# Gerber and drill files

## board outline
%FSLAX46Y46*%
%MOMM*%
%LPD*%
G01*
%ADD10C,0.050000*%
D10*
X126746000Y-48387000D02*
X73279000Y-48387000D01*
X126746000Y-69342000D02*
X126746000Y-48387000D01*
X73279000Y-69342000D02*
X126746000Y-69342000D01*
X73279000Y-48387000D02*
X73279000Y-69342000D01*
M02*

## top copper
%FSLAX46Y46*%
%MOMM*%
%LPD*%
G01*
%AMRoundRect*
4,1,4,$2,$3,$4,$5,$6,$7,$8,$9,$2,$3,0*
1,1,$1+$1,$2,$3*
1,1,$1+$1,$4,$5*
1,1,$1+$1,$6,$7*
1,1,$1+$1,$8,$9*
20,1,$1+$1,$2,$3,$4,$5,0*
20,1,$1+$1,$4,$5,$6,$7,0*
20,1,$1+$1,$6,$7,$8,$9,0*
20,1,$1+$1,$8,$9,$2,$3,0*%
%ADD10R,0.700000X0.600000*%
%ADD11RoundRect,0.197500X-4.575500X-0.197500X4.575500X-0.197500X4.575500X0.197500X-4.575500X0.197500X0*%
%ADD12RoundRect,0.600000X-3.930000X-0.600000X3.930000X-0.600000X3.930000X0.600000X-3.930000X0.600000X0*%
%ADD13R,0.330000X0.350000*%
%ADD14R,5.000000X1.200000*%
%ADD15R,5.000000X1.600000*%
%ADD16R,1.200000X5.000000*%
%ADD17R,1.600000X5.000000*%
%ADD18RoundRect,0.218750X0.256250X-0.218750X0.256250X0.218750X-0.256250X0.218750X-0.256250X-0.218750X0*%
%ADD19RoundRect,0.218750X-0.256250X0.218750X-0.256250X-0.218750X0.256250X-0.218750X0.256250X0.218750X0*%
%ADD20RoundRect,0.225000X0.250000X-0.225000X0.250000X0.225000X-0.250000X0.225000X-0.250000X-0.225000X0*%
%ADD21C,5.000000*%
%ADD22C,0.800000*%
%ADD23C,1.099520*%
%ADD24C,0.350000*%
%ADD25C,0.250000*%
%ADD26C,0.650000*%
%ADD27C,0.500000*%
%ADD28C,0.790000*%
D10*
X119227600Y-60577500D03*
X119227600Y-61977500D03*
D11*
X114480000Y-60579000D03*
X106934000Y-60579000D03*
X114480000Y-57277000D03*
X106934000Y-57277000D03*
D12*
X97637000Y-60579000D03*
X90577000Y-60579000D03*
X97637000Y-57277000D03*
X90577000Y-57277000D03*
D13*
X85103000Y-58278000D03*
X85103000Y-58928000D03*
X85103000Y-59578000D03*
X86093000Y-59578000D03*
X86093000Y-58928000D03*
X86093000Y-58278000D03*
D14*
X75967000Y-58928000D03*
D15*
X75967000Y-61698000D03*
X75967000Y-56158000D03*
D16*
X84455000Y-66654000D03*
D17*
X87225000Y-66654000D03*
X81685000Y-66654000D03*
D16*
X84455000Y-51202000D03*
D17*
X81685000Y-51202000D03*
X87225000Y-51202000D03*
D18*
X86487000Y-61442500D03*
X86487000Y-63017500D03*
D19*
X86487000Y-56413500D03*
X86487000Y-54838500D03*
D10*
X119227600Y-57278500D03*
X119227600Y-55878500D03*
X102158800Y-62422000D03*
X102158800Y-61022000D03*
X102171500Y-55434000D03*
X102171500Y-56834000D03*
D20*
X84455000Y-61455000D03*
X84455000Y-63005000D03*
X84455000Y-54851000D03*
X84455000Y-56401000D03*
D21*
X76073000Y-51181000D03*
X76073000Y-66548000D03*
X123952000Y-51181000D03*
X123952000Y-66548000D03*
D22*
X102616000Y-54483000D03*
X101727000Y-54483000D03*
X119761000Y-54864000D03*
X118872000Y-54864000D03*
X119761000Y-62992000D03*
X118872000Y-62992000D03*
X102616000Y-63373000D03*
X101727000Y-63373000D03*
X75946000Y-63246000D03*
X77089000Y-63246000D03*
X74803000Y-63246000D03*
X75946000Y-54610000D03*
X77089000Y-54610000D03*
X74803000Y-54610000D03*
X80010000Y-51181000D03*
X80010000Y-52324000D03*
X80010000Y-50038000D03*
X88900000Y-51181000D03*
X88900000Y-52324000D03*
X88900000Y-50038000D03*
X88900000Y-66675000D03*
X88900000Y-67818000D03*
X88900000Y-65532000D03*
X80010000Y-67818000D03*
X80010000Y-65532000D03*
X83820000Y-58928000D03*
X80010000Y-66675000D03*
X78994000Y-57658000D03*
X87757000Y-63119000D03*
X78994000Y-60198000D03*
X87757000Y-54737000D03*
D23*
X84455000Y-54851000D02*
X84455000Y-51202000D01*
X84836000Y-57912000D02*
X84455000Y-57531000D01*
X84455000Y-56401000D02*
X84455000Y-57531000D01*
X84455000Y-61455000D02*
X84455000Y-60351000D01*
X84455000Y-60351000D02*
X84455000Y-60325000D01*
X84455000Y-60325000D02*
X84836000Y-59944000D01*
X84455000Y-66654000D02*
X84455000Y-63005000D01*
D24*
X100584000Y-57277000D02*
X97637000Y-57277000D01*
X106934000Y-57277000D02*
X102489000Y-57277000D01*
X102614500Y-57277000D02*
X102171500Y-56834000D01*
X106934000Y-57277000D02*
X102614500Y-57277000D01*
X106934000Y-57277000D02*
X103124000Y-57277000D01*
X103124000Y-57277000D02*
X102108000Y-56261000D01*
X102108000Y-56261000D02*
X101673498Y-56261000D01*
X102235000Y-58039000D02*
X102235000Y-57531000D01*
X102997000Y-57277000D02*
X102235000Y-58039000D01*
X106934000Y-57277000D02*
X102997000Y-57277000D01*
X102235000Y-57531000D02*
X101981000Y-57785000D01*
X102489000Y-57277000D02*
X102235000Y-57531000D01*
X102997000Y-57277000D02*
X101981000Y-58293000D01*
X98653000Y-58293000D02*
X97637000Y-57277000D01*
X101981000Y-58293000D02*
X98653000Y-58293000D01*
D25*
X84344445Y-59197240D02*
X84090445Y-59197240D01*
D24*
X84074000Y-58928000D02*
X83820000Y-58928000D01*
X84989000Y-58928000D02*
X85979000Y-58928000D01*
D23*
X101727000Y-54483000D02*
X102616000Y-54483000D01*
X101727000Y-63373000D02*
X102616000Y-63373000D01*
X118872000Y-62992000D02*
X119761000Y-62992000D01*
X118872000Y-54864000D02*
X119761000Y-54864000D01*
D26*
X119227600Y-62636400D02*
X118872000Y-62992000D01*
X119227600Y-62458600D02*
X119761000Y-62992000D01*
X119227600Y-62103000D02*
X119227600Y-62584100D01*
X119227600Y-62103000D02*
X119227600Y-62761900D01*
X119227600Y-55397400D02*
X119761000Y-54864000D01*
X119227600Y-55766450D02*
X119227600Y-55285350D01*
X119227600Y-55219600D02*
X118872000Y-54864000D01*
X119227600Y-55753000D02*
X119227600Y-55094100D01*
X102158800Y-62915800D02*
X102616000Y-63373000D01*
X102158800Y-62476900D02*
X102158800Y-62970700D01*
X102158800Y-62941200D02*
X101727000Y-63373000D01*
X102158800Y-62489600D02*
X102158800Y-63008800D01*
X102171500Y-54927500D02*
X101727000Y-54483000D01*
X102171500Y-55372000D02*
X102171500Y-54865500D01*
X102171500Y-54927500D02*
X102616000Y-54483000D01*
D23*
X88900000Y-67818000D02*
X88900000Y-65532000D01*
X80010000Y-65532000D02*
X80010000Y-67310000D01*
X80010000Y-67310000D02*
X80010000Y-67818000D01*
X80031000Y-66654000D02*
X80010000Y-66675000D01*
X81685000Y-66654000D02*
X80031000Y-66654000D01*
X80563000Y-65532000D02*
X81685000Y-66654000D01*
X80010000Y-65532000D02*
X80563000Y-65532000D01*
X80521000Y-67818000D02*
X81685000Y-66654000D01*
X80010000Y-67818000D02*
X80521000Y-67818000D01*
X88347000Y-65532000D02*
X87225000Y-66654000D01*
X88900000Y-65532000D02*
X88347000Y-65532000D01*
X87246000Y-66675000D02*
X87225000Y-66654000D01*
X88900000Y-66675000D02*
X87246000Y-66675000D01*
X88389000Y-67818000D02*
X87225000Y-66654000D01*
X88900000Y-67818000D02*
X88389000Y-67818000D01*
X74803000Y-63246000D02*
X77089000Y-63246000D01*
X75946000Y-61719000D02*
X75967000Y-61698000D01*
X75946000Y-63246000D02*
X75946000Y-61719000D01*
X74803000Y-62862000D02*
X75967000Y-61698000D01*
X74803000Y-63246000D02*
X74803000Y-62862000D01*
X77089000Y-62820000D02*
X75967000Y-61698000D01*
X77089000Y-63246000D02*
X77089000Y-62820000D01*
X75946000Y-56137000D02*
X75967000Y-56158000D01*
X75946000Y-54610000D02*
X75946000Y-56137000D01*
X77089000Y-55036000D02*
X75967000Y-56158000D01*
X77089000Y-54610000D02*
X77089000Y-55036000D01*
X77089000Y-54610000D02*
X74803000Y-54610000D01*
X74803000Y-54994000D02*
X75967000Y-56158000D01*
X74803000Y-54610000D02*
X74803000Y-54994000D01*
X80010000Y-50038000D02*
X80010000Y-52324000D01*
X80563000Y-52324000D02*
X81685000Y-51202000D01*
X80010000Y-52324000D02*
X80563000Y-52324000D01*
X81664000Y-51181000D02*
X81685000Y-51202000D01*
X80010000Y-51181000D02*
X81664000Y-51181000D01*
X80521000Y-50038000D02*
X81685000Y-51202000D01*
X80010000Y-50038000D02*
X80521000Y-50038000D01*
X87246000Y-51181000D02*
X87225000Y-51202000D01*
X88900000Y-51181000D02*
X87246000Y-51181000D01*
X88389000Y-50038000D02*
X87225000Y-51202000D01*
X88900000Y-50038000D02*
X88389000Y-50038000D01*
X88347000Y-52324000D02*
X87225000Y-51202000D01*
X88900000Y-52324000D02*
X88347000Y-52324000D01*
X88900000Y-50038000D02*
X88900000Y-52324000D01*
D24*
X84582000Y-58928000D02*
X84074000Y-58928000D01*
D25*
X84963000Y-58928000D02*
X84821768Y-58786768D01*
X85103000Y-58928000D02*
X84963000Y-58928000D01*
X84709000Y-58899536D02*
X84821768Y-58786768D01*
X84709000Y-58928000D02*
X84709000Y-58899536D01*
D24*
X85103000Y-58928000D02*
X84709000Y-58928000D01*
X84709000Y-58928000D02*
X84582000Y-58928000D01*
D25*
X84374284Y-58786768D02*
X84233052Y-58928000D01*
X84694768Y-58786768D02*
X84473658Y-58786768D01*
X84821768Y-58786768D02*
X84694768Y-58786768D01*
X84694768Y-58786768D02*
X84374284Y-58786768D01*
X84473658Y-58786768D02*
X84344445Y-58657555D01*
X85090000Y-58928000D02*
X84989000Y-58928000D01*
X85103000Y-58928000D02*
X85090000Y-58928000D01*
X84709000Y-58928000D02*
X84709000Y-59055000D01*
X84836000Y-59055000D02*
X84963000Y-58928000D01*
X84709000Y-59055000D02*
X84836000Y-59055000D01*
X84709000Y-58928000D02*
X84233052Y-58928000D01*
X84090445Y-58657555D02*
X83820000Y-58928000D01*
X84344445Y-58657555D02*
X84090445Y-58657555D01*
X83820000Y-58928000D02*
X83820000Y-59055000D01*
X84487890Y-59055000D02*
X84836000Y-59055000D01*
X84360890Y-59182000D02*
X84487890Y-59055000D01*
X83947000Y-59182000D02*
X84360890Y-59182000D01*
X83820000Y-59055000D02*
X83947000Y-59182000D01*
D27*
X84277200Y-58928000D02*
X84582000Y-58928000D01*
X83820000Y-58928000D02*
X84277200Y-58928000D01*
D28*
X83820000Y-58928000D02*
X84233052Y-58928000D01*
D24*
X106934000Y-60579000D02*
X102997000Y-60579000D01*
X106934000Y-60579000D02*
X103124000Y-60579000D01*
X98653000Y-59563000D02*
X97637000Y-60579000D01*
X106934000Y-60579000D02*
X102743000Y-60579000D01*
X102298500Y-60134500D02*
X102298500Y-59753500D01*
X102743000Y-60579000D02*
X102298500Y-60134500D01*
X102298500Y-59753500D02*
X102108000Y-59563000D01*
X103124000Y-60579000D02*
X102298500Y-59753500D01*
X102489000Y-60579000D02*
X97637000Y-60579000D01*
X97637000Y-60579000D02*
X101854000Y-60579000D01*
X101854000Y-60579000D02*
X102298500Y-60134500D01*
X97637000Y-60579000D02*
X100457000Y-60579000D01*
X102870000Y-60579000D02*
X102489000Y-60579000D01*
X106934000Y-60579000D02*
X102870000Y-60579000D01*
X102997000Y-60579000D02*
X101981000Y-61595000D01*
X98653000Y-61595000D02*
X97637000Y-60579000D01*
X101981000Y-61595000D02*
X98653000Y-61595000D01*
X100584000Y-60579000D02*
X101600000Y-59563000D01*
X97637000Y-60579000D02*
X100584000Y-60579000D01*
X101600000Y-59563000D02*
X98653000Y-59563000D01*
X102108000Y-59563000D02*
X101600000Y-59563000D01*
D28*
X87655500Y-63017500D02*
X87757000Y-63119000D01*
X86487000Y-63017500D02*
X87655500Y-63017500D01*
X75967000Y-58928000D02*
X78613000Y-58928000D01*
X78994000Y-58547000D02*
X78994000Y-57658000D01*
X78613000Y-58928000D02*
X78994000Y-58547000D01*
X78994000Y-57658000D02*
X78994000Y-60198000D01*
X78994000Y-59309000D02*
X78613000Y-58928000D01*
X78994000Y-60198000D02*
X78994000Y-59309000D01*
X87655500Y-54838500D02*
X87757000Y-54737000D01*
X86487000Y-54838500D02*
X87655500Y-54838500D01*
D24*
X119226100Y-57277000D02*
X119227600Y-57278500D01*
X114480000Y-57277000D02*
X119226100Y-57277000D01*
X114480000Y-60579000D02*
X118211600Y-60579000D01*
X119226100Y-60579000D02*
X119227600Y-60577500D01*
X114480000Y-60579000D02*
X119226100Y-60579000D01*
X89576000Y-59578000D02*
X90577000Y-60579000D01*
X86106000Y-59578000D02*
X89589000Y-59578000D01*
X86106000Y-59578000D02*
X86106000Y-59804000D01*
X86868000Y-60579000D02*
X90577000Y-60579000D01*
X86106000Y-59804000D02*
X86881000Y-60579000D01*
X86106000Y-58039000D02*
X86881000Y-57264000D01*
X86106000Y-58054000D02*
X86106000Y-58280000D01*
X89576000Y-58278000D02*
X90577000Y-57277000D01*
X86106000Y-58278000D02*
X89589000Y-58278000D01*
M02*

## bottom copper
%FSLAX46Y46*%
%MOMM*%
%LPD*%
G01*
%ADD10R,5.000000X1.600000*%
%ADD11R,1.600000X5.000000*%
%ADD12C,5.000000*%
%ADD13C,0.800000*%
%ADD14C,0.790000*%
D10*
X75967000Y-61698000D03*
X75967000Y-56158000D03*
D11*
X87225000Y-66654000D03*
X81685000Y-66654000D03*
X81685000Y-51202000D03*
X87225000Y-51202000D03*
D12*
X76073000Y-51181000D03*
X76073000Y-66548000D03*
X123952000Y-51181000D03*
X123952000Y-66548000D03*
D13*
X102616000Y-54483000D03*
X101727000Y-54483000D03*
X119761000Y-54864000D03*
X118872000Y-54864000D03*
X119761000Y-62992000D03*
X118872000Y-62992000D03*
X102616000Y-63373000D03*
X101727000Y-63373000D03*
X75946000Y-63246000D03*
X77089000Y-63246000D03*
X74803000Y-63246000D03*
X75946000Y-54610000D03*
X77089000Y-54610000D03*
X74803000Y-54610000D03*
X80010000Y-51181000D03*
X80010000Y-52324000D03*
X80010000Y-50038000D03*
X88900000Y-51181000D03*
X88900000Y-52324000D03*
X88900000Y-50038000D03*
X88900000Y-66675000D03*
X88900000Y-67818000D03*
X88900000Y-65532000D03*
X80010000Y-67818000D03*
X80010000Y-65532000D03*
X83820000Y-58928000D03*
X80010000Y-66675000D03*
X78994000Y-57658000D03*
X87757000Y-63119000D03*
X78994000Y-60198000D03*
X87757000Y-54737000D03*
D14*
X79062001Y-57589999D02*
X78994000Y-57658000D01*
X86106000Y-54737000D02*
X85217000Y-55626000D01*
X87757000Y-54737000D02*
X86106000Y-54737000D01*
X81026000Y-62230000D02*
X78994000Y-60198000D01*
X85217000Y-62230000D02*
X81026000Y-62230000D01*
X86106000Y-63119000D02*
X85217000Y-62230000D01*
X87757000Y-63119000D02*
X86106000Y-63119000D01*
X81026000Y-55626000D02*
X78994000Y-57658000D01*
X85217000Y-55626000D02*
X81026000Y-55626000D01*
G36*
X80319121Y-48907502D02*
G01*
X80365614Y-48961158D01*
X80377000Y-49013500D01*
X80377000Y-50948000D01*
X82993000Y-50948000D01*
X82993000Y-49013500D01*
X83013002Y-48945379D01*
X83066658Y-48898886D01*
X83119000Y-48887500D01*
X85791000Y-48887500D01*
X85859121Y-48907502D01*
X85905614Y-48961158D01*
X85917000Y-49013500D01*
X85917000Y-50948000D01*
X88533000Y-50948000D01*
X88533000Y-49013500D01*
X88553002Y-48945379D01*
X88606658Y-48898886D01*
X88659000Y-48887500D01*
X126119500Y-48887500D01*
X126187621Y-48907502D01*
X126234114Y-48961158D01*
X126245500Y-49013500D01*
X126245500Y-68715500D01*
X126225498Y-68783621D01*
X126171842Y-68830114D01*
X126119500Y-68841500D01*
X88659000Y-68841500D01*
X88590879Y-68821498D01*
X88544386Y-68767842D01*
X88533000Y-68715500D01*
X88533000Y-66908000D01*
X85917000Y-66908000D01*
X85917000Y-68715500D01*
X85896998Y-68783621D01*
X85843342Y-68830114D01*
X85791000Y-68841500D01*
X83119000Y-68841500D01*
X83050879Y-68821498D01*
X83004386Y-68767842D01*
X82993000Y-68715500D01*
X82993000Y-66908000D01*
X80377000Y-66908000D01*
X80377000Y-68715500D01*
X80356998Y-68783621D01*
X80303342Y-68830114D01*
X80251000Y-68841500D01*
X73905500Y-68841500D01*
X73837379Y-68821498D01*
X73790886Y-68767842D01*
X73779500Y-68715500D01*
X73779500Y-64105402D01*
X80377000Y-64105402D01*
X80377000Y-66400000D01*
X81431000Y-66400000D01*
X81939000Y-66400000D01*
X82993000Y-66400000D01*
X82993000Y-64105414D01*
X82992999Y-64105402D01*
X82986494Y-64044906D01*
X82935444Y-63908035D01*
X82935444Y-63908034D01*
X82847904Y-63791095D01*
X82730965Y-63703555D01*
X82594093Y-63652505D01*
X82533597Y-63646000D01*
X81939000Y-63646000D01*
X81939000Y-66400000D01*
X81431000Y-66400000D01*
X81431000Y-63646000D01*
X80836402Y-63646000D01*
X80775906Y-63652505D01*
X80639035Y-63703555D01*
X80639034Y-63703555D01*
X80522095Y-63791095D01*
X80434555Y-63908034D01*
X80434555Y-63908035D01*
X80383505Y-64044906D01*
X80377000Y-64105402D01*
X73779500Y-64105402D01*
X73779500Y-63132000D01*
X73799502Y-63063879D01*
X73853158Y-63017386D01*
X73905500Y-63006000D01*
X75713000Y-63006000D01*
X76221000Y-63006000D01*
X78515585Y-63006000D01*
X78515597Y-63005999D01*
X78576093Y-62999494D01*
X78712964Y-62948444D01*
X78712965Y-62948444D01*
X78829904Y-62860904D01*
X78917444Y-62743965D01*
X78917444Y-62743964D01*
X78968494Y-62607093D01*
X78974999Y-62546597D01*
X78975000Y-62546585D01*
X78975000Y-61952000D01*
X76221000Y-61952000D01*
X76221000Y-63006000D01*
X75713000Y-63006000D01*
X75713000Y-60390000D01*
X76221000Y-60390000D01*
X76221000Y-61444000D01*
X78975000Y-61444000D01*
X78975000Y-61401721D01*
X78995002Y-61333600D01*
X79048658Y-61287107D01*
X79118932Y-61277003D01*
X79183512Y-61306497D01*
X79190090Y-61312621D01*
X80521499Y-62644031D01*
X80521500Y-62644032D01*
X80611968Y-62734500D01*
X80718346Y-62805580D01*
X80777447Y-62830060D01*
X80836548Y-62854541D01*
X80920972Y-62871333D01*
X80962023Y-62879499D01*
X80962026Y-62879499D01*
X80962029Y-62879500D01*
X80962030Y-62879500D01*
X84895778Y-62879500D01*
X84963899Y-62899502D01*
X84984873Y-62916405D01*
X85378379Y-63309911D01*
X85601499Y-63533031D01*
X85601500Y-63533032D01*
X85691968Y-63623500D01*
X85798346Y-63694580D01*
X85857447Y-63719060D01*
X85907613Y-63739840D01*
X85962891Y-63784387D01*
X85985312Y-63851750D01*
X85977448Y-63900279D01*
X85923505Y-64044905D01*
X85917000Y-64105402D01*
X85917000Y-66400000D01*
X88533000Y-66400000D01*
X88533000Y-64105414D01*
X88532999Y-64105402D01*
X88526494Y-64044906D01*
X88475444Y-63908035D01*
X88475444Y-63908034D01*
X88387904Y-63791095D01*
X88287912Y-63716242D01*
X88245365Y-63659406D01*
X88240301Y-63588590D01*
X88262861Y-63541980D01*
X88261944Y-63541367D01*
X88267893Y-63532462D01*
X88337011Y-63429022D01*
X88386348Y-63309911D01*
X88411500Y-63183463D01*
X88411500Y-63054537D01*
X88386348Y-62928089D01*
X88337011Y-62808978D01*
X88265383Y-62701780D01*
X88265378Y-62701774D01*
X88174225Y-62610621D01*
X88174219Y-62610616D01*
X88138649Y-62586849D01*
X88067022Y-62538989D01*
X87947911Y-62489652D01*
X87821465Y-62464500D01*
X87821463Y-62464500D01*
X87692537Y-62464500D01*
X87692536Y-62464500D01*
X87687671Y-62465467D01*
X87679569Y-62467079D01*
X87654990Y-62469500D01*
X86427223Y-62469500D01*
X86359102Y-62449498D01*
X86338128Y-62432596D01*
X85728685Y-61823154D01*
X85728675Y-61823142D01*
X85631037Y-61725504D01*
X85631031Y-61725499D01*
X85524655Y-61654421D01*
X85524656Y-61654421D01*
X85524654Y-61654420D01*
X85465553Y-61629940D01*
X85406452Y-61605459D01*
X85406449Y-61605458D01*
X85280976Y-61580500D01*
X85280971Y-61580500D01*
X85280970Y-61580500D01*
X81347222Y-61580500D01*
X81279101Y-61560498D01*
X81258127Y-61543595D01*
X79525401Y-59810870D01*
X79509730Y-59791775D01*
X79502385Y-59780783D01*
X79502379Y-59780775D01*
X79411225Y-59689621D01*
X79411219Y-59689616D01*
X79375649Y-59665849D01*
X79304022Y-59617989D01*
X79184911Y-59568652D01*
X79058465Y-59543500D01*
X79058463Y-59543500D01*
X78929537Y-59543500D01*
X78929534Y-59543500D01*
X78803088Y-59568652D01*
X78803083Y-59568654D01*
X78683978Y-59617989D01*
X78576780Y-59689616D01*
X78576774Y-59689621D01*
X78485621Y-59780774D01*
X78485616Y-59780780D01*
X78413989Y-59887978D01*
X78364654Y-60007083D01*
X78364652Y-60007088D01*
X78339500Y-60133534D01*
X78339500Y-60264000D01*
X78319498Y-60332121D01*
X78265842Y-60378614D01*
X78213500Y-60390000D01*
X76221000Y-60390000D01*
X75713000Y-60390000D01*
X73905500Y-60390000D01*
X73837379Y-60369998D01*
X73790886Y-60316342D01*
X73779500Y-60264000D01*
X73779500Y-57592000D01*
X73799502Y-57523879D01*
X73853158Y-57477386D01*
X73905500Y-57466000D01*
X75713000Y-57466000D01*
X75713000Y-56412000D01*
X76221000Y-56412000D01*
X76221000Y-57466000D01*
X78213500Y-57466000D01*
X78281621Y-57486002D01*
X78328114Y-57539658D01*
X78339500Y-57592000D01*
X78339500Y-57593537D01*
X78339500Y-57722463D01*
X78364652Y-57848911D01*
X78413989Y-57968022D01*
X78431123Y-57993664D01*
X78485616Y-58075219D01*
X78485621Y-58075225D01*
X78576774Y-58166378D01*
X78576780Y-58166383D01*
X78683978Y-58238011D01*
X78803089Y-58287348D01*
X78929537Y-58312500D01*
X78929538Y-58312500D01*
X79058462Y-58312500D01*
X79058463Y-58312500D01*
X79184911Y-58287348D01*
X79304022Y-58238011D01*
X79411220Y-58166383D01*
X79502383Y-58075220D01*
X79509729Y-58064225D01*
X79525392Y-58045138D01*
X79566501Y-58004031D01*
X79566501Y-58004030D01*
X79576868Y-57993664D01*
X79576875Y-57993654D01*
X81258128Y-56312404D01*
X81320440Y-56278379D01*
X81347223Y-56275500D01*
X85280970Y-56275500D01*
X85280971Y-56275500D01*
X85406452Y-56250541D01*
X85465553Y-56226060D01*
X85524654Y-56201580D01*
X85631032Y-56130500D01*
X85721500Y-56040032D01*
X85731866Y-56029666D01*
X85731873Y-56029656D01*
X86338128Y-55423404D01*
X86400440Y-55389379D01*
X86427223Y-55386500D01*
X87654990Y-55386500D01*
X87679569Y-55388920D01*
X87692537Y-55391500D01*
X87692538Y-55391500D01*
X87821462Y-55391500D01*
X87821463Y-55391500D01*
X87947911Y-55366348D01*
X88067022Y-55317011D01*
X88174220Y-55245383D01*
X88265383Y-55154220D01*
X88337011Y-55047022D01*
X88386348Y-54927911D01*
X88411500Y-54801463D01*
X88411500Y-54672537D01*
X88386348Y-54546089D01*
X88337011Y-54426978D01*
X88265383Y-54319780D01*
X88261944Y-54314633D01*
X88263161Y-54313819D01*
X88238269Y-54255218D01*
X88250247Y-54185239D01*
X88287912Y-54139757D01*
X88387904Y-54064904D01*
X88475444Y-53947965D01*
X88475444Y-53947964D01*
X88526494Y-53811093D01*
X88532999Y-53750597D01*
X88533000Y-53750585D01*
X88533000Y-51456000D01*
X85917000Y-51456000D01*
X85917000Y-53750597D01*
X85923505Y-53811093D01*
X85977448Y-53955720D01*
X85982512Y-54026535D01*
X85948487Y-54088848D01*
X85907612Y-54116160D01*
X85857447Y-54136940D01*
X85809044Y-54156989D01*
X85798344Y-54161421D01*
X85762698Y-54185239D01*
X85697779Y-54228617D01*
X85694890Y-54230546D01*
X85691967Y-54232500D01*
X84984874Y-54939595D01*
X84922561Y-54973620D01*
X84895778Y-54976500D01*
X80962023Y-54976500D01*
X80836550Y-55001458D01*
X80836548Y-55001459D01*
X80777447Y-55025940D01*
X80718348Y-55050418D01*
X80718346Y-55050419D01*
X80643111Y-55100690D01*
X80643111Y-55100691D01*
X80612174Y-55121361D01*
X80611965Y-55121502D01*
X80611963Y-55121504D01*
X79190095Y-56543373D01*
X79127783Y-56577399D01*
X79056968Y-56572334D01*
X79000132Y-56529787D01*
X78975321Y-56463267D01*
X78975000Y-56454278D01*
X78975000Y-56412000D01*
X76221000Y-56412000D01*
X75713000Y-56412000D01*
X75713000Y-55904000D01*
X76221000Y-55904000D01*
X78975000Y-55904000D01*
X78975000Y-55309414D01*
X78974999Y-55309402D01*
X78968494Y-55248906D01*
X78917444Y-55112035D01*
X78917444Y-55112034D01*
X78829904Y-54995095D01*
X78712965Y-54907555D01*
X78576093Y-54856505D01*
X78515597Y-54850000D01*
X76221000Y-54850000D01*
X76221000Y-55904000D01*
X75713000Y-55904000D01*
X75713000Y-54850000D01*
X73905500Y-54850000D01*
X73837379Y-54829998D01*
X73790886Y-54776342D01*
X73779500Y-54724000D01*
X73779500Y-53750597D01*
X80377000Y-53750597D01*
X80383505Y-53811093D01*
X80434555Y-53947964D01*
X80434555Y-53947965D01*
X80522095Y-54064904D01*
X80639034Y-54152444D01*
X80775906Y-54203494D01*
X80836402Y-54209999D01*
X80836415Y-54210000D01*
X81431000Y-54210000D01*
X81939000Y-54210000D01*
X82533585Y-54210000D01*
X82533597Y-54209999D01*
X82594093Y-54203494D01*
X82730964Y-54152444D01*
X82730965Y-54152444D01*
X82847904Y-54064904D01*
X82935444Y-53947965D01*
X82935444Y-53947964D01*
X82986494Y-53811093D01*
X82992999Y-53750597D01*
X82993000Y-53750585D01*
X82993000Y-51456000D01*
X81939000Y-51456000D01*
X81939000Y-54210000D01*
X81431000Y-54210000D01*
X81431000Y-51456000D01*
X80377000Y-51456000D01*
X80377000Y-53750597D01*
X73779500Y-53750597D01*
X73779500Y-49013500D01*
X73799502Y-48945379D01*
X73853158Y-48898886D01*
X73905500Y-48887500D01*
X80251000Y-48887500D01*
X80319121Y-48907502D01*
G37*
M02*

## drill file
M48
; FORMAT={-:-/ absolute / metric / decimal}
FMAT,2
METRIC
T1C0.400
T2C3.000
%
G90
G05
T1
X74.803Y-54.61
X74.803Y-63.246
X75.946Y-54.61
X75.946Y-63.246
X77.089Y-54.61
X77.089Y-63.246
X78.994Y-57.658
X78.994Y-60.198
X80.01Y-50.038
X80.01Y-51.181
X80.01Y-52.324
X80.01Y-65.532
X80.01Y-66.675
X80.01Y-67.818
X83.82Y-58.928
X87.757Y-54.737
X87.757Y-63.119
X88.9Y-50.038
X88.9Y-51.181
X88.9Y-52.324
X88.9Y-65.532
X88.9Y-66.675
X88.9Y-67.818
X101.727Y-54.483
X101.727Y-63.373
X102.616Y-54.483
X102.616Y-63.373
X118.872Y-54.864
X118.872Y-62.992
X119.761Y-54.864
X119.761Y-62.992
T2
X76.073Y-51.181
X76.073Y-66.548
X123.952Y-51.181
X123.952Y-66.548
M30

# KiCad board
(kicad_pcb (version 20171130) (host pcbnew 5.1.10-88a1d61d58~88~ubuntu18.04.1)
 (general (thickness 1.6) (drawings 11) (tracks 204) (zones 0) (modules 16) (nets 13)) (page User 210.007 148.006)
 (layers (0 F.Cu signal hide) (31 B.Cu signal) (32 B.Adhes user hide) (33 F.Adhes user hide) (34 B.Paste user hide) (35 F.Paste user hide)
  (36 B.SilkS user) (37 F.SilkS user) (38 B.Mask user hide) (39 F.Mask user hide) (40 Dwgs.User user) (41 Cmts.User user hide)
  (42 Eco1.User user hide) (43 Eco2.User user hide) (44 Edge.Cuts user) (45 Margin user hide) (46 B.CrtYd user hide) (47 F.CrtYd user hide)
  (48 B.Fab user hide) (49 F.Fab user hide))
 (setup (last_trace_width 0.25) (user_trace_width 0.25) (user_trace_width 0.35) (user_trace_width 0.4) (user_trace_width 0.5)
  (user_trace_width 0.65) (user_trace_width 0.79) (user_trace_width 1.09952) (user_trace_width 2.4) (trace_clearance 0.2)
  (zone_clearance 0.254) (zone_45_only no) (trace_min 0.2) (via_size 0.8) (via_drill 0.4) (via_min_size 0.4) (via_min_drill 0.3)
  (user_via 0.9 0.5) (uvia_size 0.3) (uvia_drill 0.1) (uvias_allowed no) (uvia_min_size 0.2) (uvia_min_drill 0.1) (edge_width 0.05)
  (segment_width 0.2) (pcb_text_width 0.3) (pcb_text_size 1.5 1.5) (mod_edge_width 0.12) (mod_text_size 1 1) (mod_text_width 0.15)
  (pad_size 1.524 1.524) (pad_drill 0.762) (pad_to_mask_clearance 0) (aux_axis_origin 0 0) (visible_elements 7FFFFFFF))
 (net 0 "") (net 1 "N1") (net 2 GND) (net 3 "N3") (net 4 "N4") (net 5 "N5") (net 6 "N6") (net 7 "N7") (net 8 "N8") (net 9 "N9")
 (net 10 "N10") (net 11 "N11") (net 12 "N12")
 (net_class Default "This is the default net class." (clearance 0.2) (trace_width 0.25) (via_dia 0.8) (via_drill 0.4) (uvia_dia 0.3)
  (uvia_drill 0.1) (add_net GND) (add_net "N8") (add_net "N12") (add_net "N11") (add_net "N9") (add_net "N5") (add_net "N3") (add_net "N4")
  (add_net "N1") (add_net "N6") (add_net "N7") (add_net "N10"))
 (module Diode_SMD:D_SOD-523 (layer F.Cu) (at 119.2276 61.2775 270)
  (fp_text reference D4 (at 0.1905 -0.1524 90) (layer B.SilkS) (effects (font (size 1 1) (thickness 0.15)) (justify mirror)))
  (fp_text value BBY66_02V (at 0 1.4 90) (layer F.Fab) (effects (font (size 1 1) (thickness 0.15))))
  (pad 1 smd rect (at -0.7 0 90) (size 0.6 0.7) (layers F.Cu F.Paste F.Mask) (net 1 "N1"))
  (pad 2 smd rect (at 0.7 0 90) (size 0.6 0.7) (layers F.Cu F.Paste F.Mask) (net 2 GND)))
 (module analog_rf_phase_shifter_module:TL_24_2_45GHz (layer F.Cu) (at 110.707 60.579)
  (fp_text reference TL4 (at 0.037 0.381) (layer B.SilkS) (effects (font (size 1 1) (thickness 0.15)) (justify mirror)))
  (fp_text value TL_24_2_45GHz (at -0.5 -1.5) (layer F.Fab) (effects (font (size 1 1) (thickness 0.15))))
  (pad 2 smd roundrect (at 3.773 0) (size 9.546 0.79) (layers F.Cu F.Mask) (roundrect_rratio 0.25) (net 1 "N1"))
  (pad 1 smd roundrect (at -3.773 0) (size 9.546 0.79) (layers F.Cu F.Mask) (roundrect_rratio 0.25) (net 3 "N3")))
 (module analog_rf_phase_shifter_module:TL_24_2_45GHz (layer F.Cu) (at 110.707 57.277)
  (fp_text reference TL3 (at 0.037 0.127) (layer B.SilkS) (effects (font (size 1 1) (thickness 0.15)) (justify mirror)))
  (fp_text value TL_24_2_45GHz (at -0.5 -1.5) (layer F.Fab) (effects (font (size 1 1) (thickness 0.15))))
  (pad 2 smd roundrect (at 3.773 0) (size 9.546 0.79) (layers F.Cu F.Mask) (roundrect_rratio 0.25) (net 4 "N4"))
  (pad 1 smd roundrect (at -3.773 0) (size 9.546 0.79) (layers F.Cu F.Mask) (roundrect_rratio 0.25) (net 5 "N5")))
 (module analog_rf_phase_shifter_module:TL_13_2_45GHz (layer F.Cu) (at 94.107 60.579)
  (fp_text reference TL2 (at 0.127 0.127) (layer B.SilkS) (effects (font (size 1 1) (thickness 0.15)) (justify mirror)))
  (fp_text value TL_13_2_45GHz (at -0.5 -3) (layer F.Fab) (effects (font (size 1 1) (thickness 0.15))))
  (pad 2 smd roundrect (at 3.53 0) (size 9.06 2.4) (layers F.Cu F.Mask) (roundrect_rratio 0.25) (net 3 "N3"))
  (pad 1 smd roundrect (at -3.53 0) (size 9.06 2.4) (layers F.Cu F.Mask) (roundrect_rratio 0.25) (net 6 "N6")))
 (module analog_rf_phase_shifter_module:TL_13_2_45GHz (layer F.Cu) (at 94.107 57.277)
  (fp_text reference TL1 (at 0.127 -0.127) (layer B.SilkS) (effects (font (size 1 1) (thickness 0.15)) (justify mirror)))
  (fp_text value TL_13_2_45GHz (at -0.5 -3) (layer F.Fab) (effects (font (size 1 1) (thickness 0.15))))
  (pad 2 smd roundrect (at 3.53 0) (size 9.06 2.4) (layers F.Cu F.Mask) (roundrect_rratio 0.25) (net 5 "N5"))
  (pad 1 smd roundrect (at -3.53 0) (size 9.06 2.4) (layers F.Cu F.Mask) (roundrect_rratio 0.25) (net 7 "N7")))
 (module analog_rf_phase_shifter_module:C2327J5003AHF (layer F.Cu) (at 85.598 58.928 270)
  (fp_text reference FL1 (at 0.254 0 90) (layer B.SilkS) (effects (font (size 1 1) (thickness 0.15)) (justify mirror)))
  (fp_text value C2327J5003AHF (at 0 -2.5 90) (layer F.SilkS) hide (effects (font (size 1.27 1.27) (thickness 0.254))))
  (pad 1 smd rect (at -0.65 0.495) (size 0.33 0.35) (layers F.Cu F.Paste F.Mask) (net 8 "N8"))
  (pad 2 smd rect (at 0 0.495) (size 0.33 0.35) (layers F.Cu F.Paste F.Mask) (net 2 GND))
  (pad 3 smd rect (at 0.65 0.495) (size 0.33 0.35) (layers F.Cu F.Paste F.Mask) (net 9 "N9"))
  (pad 4 smd rect (at 0.65 -0.495) (size 0.33 0.35) (layers F.Cu F.Paste F.Mask) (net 6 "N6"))
  (pad 5 smd rect (at 0 -0.495) (size 0.33 0.35) (layers F.Cu F.Paste F.Mask) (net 2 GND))
  (pad 6 smd rect (at -0.65 -0.495) (size 0.33 0.35) (layers F.Cu F.Paste F.Mask) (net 7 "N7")))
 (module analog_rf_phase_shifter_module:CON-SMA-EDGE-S (layer F.Cu) (at 68.707 58.928 90)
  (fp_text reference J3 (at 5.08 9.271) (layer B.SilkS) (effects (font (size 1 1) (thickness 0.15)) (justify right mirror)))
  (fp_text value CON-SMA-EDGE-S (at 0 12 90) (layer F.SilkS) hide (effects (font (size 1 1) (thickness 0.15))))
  (pad 1 smd rect (at 0 7.26 90) (size 1.2 5) (layers F.Cu F.Paste F.Mask) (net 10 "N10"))
  (pad 2 smd rect (at -2.77 7.26 90) (size 1.6 5) (layers F.Cu F.Paste F.Mask) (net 2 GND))
  (pad 2 smd rect (at 2.77 7.26 90) (size 1.6 5) (layers F.Cu F.Paste F.Mask) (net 2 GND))
  (pad 2 smd rect (at -2.77 7.26 90) (size 1.6 5) (layers B.Cu B.Paste B.Mask) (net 2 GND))
  (pad 2 smd rect (at 2.77 7.26 90) (size 1.6 5) (layers B.Cu B.Paste B.Mask) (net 2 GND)))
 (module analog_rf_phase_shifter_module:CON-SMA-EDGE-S (layer F.Cu) (at 84.455 73.914 180)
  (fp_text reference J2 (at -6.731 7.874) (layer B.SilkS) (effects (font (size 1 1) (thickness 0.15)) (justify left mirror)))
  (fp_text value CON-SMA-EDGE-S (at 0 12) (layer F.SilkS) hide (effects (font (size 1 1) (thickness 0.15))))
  (pad 1 smd rect (at 0 7.26 180) (size 1.2 5) (layers F.Cu F.Paste F.Mask) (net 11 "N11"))
  (pad 2 smd rect (at -2.77 7.26 180) (size 1.6 5) (layers F.Cu F.Paste F.Mask) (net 2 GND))
  (pad 2 smd rect (at 2.77 7.26 180) (size 1.6 5) (layers F.Cu F.Paste F.Mask) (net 2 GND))
  (pad 2 smd rect (at -2.77 7.26 180) (size 1.6 5) (layers B.Cu B.Paste B.Mask) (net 2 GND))
  (pad 2 smd rect (at 2.77 7.26 180) (size 1.6 5) (layers B.Cu B.Paste B.Mask) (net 2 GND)))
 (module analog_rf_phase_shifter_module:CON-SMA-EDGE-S (layer F.Cu) (at 84.455 43.942)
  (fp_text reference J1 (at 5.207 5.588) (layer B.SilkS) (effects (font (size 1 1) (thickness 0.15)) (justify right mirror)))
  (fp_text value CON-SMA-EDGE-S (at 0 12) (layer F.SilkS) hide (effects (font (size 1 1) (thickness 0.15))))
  (pad 1 smd rect (at 0 7.26) (size 1.2 5) (layers F.Cu F.Paste F.Mask) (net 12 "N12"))
  (pad 2 smd rect (at -2.77 7.26) (size 1.6 5) (layers F.Cu F.Paste F.Mask) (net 2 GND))
  (pad 2 smd rect (at 2.77 7.26) (size 1.6 5) (layers F.Cu F.Paste F.Mask) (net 2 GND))
  (pad 2 smd rect (at -2.77 7.26) (size 1.6 5) (layers B.Cu B.Paste B.Mask) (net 2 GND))
  (pad 2 smd rect (at 2.77 7.26) (size 1.6 5) (layers B.Cu B.Paste B.Mask) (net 2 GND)))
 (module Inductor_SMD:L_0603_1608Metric (layer F.Cu) (at 86.487 62.23 90)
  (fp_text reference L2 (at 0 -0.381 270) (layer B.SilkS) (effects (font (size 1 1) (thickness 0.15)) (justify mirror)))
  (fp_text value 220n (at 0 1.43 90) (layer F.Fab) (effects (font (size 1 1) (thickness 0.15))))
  (pad 2 smd roundrect (at 0.7875 0 90) (size 0.875 0.95) (layers F.Cu F.Paste F.Mask) (roundrect_rratio 0.25) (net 6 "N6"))
  (pad 1 smd roundrect (at -0.7875 0 90) (size 0.875 0.95) (layers F.Cu F.Paste F.Mask) (roundrect_rratio 0.25) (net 10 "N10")))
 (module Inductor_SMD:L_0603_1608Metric (layer F.Cu) (at 86.487 55.626 270)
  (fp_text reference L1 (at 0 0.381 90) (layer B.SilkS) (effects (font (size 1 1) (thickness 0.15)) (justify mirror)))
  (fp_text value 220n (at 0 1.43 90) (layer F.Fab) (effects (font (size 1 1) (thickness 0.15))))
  (pad 2 smd roundrect (at 0.7875 0 270) (size 0.875 0.95) (layers F.Cu F.Paste F.Mask) (roundrect_rratio 0.25) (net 7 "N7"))
  (pad 1 smd roundrect (at -0.7875 0 270) (size 0.875 0.95) (layers F.Cu F.Paste F.Mask) (roundrect_rratio 0.25) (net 10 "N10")))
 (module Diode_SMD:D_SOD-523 (layer F.Cu) (at 119.2276 56.5785 90)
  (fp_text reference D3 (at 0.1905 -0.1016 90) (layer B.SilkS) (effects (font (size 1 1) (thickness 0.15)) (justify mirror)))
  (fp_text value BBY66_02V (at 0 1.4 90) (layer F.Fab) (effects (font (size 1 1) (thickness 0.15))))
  (pad 1 smd rect (at -0.7 0 270) (size 0.6 0.7) (layers F.Cu F.Paste F.Mask) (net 4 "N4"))
  (pad 2 smd rect (at 0.7 0 270) (size 0.6 0.7) (layers F.Cu F.Paste F.Mask) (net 2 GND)))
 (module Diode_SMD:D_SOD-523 (layer F.Cu) (at 102.1588 61.722 270)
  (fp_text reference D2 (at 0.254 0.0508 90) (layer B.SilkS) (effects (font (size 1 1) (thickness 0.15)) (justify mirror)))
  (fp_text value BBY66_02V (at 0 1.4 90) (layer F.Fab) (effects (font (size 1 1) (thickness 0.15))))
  (pad 2 smd rect (at 0.7 0 90) (size 0.6 0.7) (layers F.Cu F.Paste F.Mask) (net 2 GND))
  (pad 1 smd rect (at -0.7 0 90) (size 0.6 0.7) (layers F.Cu F.Paste F.Mask) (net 3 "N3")))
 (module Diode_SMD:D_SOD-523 (layer F.Cu) (at 102.1715 56.134 90)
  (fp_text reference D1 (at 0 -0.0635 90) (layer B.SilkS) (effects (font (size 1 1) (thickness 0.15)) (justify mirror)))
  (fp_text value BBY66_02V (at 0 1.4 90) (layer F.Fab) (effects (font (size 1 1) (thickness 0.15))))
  (pad 2 smd rect (at 0.7 0 270) (size 0.6 0.7) (layers F.Cu F.Paste F.Mask) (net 2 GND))
  (pad 1 smd rect (at -0.7 0 270) (size 0.6 0.7) (layers F.Cu F.Paste F.Mask) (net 5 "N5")))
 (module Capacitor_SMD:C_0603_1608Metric (layer F.Cu) (at 84.455 62.23 90)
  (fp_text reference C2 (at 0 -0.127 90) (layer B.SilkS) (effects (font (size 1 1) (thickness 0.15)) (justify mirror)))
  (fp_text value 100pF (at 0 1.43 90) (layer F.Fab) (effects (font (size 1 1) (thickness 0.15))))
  (pad 2 smd roundrect (at 0.775 0 90) (size 0.9 0.95) (layers F.Cu F.Paste F.Mask) (roundrect_rratio 0.25) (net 9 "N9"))
  (pad 1 smd roundrect (at -0.775 0 90) (size 0.9 0.95) (layers F.Cu F.Paste F.Mask) (roundrect_rratio 0.25) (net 11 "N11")))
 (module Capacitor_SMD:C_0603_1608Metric (layer F.Cu) (at 84.455 55.626 90)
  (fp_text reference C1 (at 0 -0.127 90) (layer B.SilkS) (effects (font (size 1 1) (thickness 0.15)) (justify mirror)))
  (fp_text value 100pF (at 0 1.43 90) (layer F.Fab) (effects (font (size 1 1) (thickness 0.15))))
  (pad 2 smd roundrect (at 0.775 0 90) (size 0.9 0.95) (layers F.Cu F.Paste F.Mask) (roundrect_rratio 0.25) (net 12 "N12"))
  (pad 1 smd roundrect (at -0.775 0 90) (size 0.9 0.95) (layers F.Cu F.Paste F.Mask) (roundrect_rratio 0.25) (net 8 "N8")))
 (gr_line (start 126.746 48.387) (end 73.279 48.387) (layer Edge.Cuts) (width 0.05))
 (gr_line (start 126.746 69.342) (end 126.746 48.387) (layer Edge.Cuts) (width 0.05))
 (gr_line (start 73.279 69.342) (end 126.746 69.342) (layer Edge.Cuts) (width 0.05))
 (gr_line (start 73.279 48.387) (end 73.279 69.342) (layer Edge.Cuts) (width 0.05))
 (segment (start 84.455 54.851) (end 84.455 51.202) (width 1.09952) (layer F.Cu) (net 12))
 (segment (start 84.836 57.912) (end 84.455 57.531) (width 1.09952) (layer F.Cu) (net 8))
 (segment (start 84.455 56.401) (end 84.455 57.531) (width 1.09952) (layer F.Cu) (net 8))
 (segment (start 84.455 61.455) (end 84.455 60.351) (width 1.09952) (layer F.Cu) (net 9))
 (segment (start 84.455 60.351) (end 84.455 60.325) (width 1.09952) (layer F.Cu) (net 9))
 (segment (start 84.455 60.325) (end 84.836 59.944) (width 1.09952) (layer F.Cu) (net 9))
 (segment (start 84.455 66.654) (end 84.455 63.005) (width 1.09952) (layer F.Cu) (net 11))
 (segment (start 100.584 57.277) (end 97.637 57.277) (width 0.35) (layer F.Cu) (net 5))
 (segment (start 106.934 57.277) (end 102.489 57.277) (width 0.35) (layer F.Cu) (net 5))
 (segment (start 102.6145 57.277) (end 102.1715 56.834) (width 0.35) (layer F.Cu) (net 5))
 (segment (start 106.934 57.277) (end 102.6145 57.277) (width 0.35) (layer F.Cu) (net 5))
 (segment (start 106.934 57.277) (end 103.124 57.277) (width 0.35) (layer F.Cu) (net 5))
 (segment (start 103.124 57.277) (end 102.108 56.261) (width 0.35) (layer F.Cu) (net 5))
 (segment (start 102.108 56.261) (end 101.673498 56.261) (width 0.35) (layer F.Cu) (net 5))
 (segment (start 102.235 58.039) (end 102.235 57.531) (width 0.35) (layer F.Cu) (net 5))
 (segment (start 102.997 57.277) (end 102.235 58.039) (width 0.35) (layer F.Cu) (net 5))
 (segment (start 106.934 57.277) (end 102.997 57.277) (width 0.35) (layer F.Cu) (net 5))
 (segment (start 102.235 57.531) (end 101.981 57.785) (width 0.35) (layer F.Cu) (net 5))
 (segment (start 102.489 57.277) (end 102.235 57.531) (width 0.35) (layer F.Cu) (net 5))
 (segment (start 102.997 57.277) (end 101.981 58.293) (width 0.35) (layer F.Cu) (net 5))
 (segment (start 98.653 58.293) (end 97.637 57.277) (width 0.35) (layer F.Cu) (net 5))
 (segment (start 101.981 58.293) (end 98.653 58.293) (width 0.35) (layer F.Cu) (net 5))
 (segment (start 84.344445 59.19724) (end 84.090445 59.19724) (width 0.25) (layer F.Cu) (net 2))
 (via (at 76.073 51.181) (size 5) (drill 3) (layers F.Cu B.Cu) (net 2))
 (via (at 76.073 66.548) (size 5) (drill 3) (layers F.Cu B.Cu) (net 2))
 (via (at 123.952 51.181) (size 5) (drill 3) (layers F.Cu B.Cu) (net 2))
 (via (at 123.952 66.548) (size 5) (drill 3) (layers F.Cu B.Cu) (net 2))
 (via (at 102.616 54.483) (size 0.8) (drill 0.4) (layers F.Cu B.Cu) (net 2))
 (via (at 101.727 54.483) (size 0.8) (drill 0.4) (layers F.Cu B.Cu) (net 2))
 (via (at 119.761 54.864) (size 0.8) (drill 0.4) (layers F.Cu B.Cu) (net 2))
 (via (at 118.872 54.864) (size 0.8) (drill 0.4) (layers F.Cu B.Cu) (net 2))
 (via (at 119.761 62.992) (size 0.8) (drill 0.4) (layers F.Cu B.Cu) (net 2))
 (via (at 118.872 62.992) (size 0.8) (drill 0.4) (layers F.Cu B.Cu) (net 2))
 (via (at 102.616 63.373) (size 0.8) (drill 0.4) (layers F.Cu B.Cu) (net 2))
 (via (at 101.727 63.373) (size 0.8) (drill 0.4) (layers F.Cu B.Cu) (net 2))
 (via (at 75.946 63.246) (size 0.8) (drill 0.4) (layers F.Cu B.Cu) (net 2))
 (via (at 77.089 63.246) (size 0.8) (drill 0.4) (layers F.Cu B.Cu) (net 2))
 (via (at 74.803 63.246) (size 0.8) (drill 0.4) (layers F.Cu B.Cu) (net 2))
 (via (at 75.946 54.61) (size 0.8) (drill 0.4) (layers F.Cu B.Cu) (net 2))
 (via (at 77.089 54.61) (size 0.8) (drill 0.4) (layers F.Cu B.Cu) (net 2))
 (via (at 74.803 54.61) (size 0.8) (drill 0.4) (layers F.Cu B.Cu) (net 2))
 (via (at 80.01 51.181) (size 0.8) (drill 0.4) (layers F.Cu B.Cu) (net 2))
 (via (at 80.01 52.324) (size 0.8) (drill 0.4) (layers F.Cu B.Cu) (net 2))
 (via (at 80.01 50.038) (size 0.8) (drill 0.4) (layers F.Cu B.Cu) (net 2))
 (via (at 88.9 51.181) (size 0.8) (drill 0.4) (layers F.Cu B.Cu) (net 2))
 (via (at 88.9 52.324) (size 0.8) (drill 0.4) (layers F.Cu B.Cu) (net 2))
 (via (at 88.9 50.038) (size 0.8) (drill 0.4) (layers F.Cu B.Cu) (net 2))
 (via (at 88.9 66.675) (size 0.8) (drill 0.4) (layers F.Cu B.Cu) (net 2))
 (via (at 88.9 67.818) (size 0.8) (drill 0.4) (layers F.Cu B.Cu) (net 2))
 (via (at 88.9 65.532) (size 0.8) (drill 0.4) (layers F.Cu B.Cu) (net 2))
 (via (at 80.01 67.818) (size 0.8) (drill 0.4) (layers F.Cu B.Cu) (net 2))
 (via (at 80.01 65.532) (size 0.8) (drill 0.4) (layers F.Cu B.Cu) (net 2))
 (via (at 83.82 58.928) (size 0.8) (drill 0.4) (layers F.Cu B.Cu) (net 2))
 (segment (start 84.074 58.928) (end 83.82 58.928) (width 0.35) (layer F.Cu) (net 2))
 (segment (start 84.989 58.928) (end 85.979 58.928) (width 0.35) (layer F.Cu) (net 2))
 (via (at 80.01 66.675) (size 0.8) (drill 0.4) (layers F.Cu B.Cu) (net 2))
 (segment (start 101.727 54.483) (end 102.616 54.483) (width 1.09952) (layer F.Cu) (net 2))
 (segment (start 101.727 63.373) (end 102.616 63.373) (width 1.09952) (layer F.Cu) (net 2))
 (segment (start 118.872 62.992) (end 119.761 62.992) (width 1.09952) (layer F.Cu) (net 2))
 (segment (start 118.872 54.864) (end 119.761 54.864) (width 1.09952) (layer F.Cu) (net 2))
 (segment (start 119.2276 62.6364) (end 118.872 62.992) (width 0.65) (layer F.Cu) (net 2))
 (segment (start 119.2276 62.4586) (end 119.761 62.992) (width 0.65) (layer F.Cu) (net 2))
 (segment (start 119.2276 62.103) (end 119.2276 62.5841) (width 0.65) (layer F.Cu) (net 2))
 (segment (start 119.2276 62.103) (end 119.2276 62.7619) (width 0.65) (layer F.Cu) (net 2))
 (segment (start 119.2276 55.3974) (end 119.761 54.864) (width 0.65) (layer F.Cu) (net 2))
 (segment (start 119.2276 55.76645) (end 119.2276 55.28535) (width 0.65) (layer F.Cu) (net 2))
 (segment (start 119.2276 55.2196) (end 118.872 54.864) (width 0.65) (layer F.Cu) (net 2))
 (segment (start 119.2276 55.753) (end 119.2276 55.0941) (width 0.65) (layer F.Cu) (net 2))
 (segment (start 102.1588 62.9158) (end 102.616 63.373) (width 0.65) (layer F.Cu) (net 2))
 (segment (start 102.1588 62.4769) (end 102.1588 62.9707) (width 0.65) (layer F.Cu) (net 2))
 (segment (start 102.1588 62.9412) (end 101.727 63.373) (width 0.65) (layer F.Cu) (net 2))
 (segment (start 102.1588 62.4896) (end 102.1588 63.0088) (width 0.65) (layer F.Cu) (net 2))
 (segment (start 102.1715 54.9275) (end 101.727 54.483) (width 0.65) (layer F.Cu) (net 2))
 (segment (start 102.1715 55.372) (end 102.1715 54.8655) (width 0.65) (layer F.Cu) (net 2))
 (segment (start 102.1715 54.9275) (end 102.616 54.483) (width 0.65) (layer F.Cu) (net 2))
 (segment (start 88.9 67.818) (end 88.9 65.532) (width 1.09952) (layer F.Cu) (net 2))
 (segment (start 80.01 65.532) (end 80.01 67.31) (width 1.09952) (layer F.Cu) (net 2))
 (segment (start 80.01 67.31) (end 80.01 67.818) (width 1.09952) (layer F.Cu) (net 2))
 (segment (start 80.031 66.654) (end 80.01 66.675) (width 1.09952) (layer F.Cu) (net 2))
 (segment (start 81.685 66.654) (end 80.031 66.654) (width 1.09952) (layer F.Cu) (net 2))
 (segment (start 80.563 65.532) (end 81.685 66.654) (width 1.09952) (layer F.Cu) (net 2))
 (segment (start 80.01 65.532) (end 80.563 65.532) (width 1.09952) (layer F.Cu) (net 2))
 (segment (start 80.521 67.818) (end 81.685 66.654) (width 1.09952) (layer F.Cu) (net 2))
 (segment (start 80.01 67.818) (end 80.521 67.818) (width 1.09952) (layer F.Cu) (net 2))
 (segment (start 88.347 65.532) (end 87.225 66.654) (width 1.09952) (layer F.Cu) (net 2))
 (segment (start 88.9 65.532) (end 88.347 65.532) (width 1.09952) (layer F.Cu) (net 2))
 (segment (start 87.246 66.675) (end 87.225 66.654) (width 1.09952) (layer F.Cu) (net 2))
 (segment (start 88.9 66.675) (end 87.246 66.675) (width 1.09952) (layer F.Cu) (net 2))
 (segment (start 88.389 67.818) (end 87.225 66.654) (width 1.09952) (layer F.Cu) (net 2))
 (segment (start 88.9 67.818) (end 88.389 67.818) (width 1.09952) (layer F.Cu) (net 2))
 (segment (start 74.803 63.246) (end 77.089 63.246) (width 1.09952) (layer F.Cu) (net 2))
 (segment (start 75.946 61.719) (end 75.967 61.698) (width 1.09952) (layer F.Cu) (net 2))
 (segment (start 75.946 63.246) (end 75.946 61.719) (width 1.09952) (layer F.Cu) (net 2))
 (segment (start 74.803 62.862) (end 75.967 61.698) (width 1.09952) (layer F.Cu) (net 2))
 (segment (start 74.803 63.246) (end 74.803 62.862) (width 1.09952) (layer F.Cu) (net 2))
 (segment (start 77.089 62.82) (end 75.967 61.698) (width 1.09952) (layer F.Cu) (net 2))
 (segment (start 77.089 63.246) (end 77.089 62.82) (width 1.09952) (layer F.Cu) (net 2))
 (segment (start 75.946 56.137) (end 75.967 56.158) (width 1.09952) (layer F.Cu) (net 2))
 (segment (start 75.946 54.61) (end 75.946 56.137) (width 1.09952) (layer F.Cu) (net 2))
 (segment (start 77.089 55.036) (end 75.967 56.158) (width 1.09952) (layer F.Cu) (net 2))
 (segment (start 77.089 54.61) (end 77.089 55.036) (width 1.09952) (layer F.Cu) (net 2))
 (segment (start 77.089 54.61) (end 74.803 54.61) (width 1.09952) (layer F.Cu) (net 2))
 (segment (start 74.803 54.994) (end 75.967 56.158) (width 1.09952) (layer F.Cu) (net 2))
 (segment (start 74.803 54.61) (end 74.803 54.994) (width 1.09952) (layer F.Cu) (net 2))
 (segment (start 80.01 50.038) (end 80.01 52.324) (width 1.09952) (layer F.Cu) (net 2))
 (segment (start 80.563 52.324) (end 81.685 51.202) (width 1.09952) (layer F.Cu) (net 2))
 (segment (start 80.01 52.324) (end 80.563 52.324) (width 1.09952) (layer F.Cu) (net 2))
 (segment (start 81.664 51.181) (end 81.685 51.202) (width 1.09952) (layer F.Cu) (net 2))
 (segment (start 80.01 51.181) (end 81.664 51.181) (width 1.09952) (layer F.Cu) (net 2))
 (segment (start 80.521 50.038) (end 81.685 51.202) (width 1.09952) (layer F.Cu) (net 2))
 (segment (start 80.01 50.038) (end 80.521 50.038) (width 1.09952) (layer F.Cu) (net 2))
 (segment (start 87.246 51.181) (end 87.225 51.202) (width 1.09952) (layer F.Cu) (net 2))
 (segment (start 88.9 51.181) (end 87.246 51.181) (width 1.09952) (layer F.Cu) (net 2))
 (segment (start 88.389 50.038) (end 87.225 51.202) (width 1.09952) (layer F.Cu) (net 2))
 (segment (start 88.9 50.038) (end 88.389 50.038) (width 1.09952) (layer F.Cu) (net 2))
 (segment (start 88.347 52.324) (end 87.225 51.202) (width 1.09952) (layer F.Cu) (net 2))
 (segment (start 88.9 52.324) (end 88.347 52.324) (width 1.09952) (layer F.Cu) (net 2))
 (segment (start 88.9 50.038) (end 88.9 52.324) (width 1.09952) (layer F.Cu) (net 2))
 (segment (start 84.582 58.928) (end 84.074 58.928) (width 0.35) (layer F.Cu) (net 2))
 (segment (start 84.963 58.928) (end 84.821768 58.786768) (width 0.25) (layer F.Cu) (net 2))
 (segment (start 85.103 58.928) (end 84.963 58.928) (width 0.25) (layer F.Cu) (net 2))
 (segment (start 84.709 58.899536) (end 84.821768 58.786768) (width 0.25) (layer F.Cu) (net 2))
 (segment (start 84.709 58.928) (end 84.709 58.899536) (width 0.25) (layer F.Cu) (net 2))
 (segment (start 85.103 58.928) (end 84.709 58.928) (width 0.35) (layer F.Cu) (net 2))
 (segment (start 84.709 58.928) (end 84.582 58.928) (width 0.35) (layer F.Cu) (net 2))
 (segment (start 84.374284 58.786768) (end 84.233052 58.928) (width 0.25) (layer F.Cu) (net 2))
 (segment (start 84.694768 58.786768) (end 84.473658 58.786768) (width 0.25) (layer F.Cu) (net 2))
 (segment (start 84.821768 58.786768) (end 84.694768 58.786768) (width 0.25) (layer F.Cu) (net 2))
 (segment (start 84.694768 58.786768) (end 84.374284 58.786768) (width 0.25) (layer F.Cu) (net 2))
 (segment (start 84.473658 58.786768) (end 84.344445 58.657555) (width 0.25) (layer F.Cu) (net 2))
 (segment (start 85.09 58.928) (end 84.989 58.928) (width 0.25) (layer F.Cu) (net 2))
 (segment (start 85.103 58.928) (end 85.09 58.928) (width 0.25) (layer F.Cu) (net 2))
 (segment (start 84.709 58.928) (end 84.709 59.055) (width 0.25) (layer F.Cu) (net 2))
 (segment (start 84.836 59.055) (end 84.963 58.928) (width 0.25) (layer F.Cu) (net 2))
 (segment (start 84.709 59.055) (end 84.836 59.055) (width 0.25) (layer F.Cu) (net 2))
 (segment (start 84.709 58.928) (end 84.233052 58.928) (width 0.25) (layer F.Cu) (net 2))
 (segment (start 84.090445 58.657555) (end 83.82 58.928) (width 0.25) (layer F.Cu) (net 2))
 (segment (start 84.344445 58.657555) (end 84.090445 58.657555) (width 0.25) (layer F.Cu) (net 2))
 (segment (start 83.82 58.928) (end 83.82 59.055) (width 0.25) (layer F.Cu) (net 2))
 (segment (start 84.48789 59.055) (end 84.836 59.055) (width 0.25) (layer F.Cu) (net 2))
 (segment (start 84.36089 59.182) (end 84.48789 59.055) (width 0.25) (layer F.Cu) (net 2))
 (segment (start 83.947 59.182) (end 84.36089 59.182) (width 0.25) (layer F.Cu) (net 2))
 (segment (start 83.82 59.055) (end 83.947 59.182) (width 0.25) (layer F.Cu) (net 2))
 (segment (start 84.2772 58.928) (end 84.582 58.928) (width 0.5) (layer F.Cu) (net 2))
 (segment (start 83.82 58.928) (end 84.2772 58.928) (width 0.5) (layer F.Cu) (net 2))
 (segment (start 83.82 58.928) (end 84.233052 58.928) (width 0.79) (layer F.Cu) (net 2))
 (segment (start 106.934 60.579) (end 102.997 60.579) (width 0.35) (layer F.Cu) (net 3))
 (segment (start 106.934 60.579) (end 103.124 60.579) (width 0.35) (layer F.Cu) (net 3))
 (segment (start 98.653 59.563) (end 97.637 60.579) (width 0.35) (layer F.Cu) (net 3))
 (segment (start 106.934 60.579) (end 102.743 60.579) (width 0.35) (layer F.Cu) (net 3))
 (segment (start 102.2985 60.1345) (end 102.2985 59.7535) (width 0.35) (layer F.Cu) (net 3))
 (segment (start 102.743 60.579) (end 102.2985 60.1345) (width 0.35) (layer F.Cu) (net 3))
 (segment (start 102.2985 59.7535) (end 102.108 59.563) (width 0.35) (layer F.Cu) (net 3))
 (segment (start 103.124 60.579) (end 102.2985 59.7535) (width 0.35) (layer F.Cu) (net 3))
 (segment (start 102.489 60.579) (end 97.637 60.579) (width 0.35) (layer F.Cu) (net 3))
 (segment (start 97.637 60.579) (end 101.854 60.579) (width 0.35) (layer F.Cu) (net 3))
 (segment (start 101.854 60.579) (end 102.2985 60.1345) (width 0.35) (layer F.Cu) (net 3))
 (segment (start 97.637 60.579) (end 100.457 60.579) (width 0.35) (layer F.Cu) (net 3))
 (segment (start 102.87 60.579) (end 102.489 60.579) (width 0.35) (layer F.Cu) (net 3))
 (segment (start 106.934 60.579) (end 102.87 60.579) (width 0.35) (layer F.Cu) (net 3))
 (segment (start 102.997 60.579) (end 101.981 61.595) (width 0.35) (layer F.Cu) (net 3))
 (segment (start 98.653 61.595) (end 97.637 60.579) (width 0.35) (layer F.Cu) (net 3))
 (segment (start 101.981 61.595) (end 98.653 61.595) (width 0.35) (layer F.Cu) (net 3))
 (segment (start 100.584 60.579) (end 101.6 59.563) (width 0.35) (layer F.Cu) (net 3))
 (segment (start 97.637 60.579) (end 100.584 60.579) (width 0.35) (layer F.Cu) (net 3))
 (segment (start 101.6 59.563) (end 98.653 59.563) (width 0.35) (layer F.Cu) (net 3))
 (segment (start 102.108 59.563) (end 101.6 59.563) (width 0.35) (layer F.Cu) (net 3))
 (via (at 78.994 57.658) (size 0.8) (drill 0.4) (layers F.Cu B.Cu) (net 10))
 (segment (start 79.062001 57.589999) (end 78.994 57.658) (width 0.79) (layer B.Cu) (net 10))
 (via (at 87.757 63.119) (size 0.8) (drill 0.4) (layers F.Cu B.Cu) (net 10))
 (segment (start 87.6555 63.0175) (end 87.757 63.119) (width 0.79) (layer F.Cu) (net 10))
 (segment (start 86.487 63.0175) (end 87.6555 63.0175) (width 0.79) (layer F.Cu) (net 10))
 (via (at 78.994 60.198) (size 0.8) (drill 0.4) (layers F.Cu B.Cu) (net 10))
 (segment (start 75.967 58.928) (end 78.613 58.928) (width 0.79) (layer F.Cu) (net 10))
 (segment (start 78.994 58.547) (end 78.994 57.658) (width 0.79) (layer F.Cu) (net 10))
 (segment (start 78.613 58.928) (end 78.994 58.547) (width 0.79) (layer F.Cu) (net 10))
 (segment (start 78.994 57.658) (end 78.994 60.198) (width 0.79) (layer F.Cu) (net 10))
 (segment (start 78.994 59.309) (end 78.613 58.928) (width 0.79) (layer F.Cu) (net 10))
 (segment (start 78.994 60.198) (end 78.994 59.309) (width 0.79) (layer F.Cu) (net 10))
 (via (at 87.757 54.737) (size 0.8) (drill 0.4) (layers F.Cu B.Cu) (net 10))
 (segment (start 87.6555 54.8385) (end 87.757 54.737) (width 0.79) (layer F.Cu) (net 10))
 (segment (start 86.487 54.8385) (end 87.6555 54.8385) (width 0.79) (layer F.Cu) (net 10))
 (segment (start 86.106 54.737) (end 85.217 55.626) (width 0.79) (layer B.Cu) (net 10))
 (segment (start 87.757 54.737) (end 86.106 54.737) (width 0.79) (layer B.Cu) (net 10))
 (segment (start 81.026 62.23) (end 78.994 60.198) (width 0.79) (layer B.Cu) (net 10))
 (segment (start 85.217 62.23) (end 81.026 62.23) (width 0.79) (layer B.Cu) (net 10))
 (segment (start 86.106 63.119) (end 85.217 62.23) (width 0.79) (layer B.Cu) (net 10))
 (segment (start 87.757 63.119) (end 86.106 63.119) (width 0.79) (layer B.Cu) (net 10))
 (segment (start 81.026 55.626) (end 78.994 57.658) (width 0.79) (layer B.Cu) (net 10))
 (segment (start 85.217 55.626) (end 81.026 55.626) (width 0.79) (layer B.Cu) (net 10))
 (segment (start 119.2261 57.277) (end 119.2276 57.2785) (width 0.35) (layer F.Cu) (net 4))
 (segment (start 114.48 57.277) (end 119.2261 57.277) (width 0.35) (layer F.Cu) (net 4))
 (segment (start 114.48 60.579) (end 118.2116 60.579) (width 0.35) (layer F.Cu) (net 1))
 (segment (start 119.2261 60.579) (end 119.2276 60.5775) (width 0.35) (layer F.Cu) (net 1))
 (segment (start 114.48 60.579) (end 119.2261 60.579) (width 0.35) (layer F.Cu) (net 1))
 (segment (start 89.576 59.578) (end 90.577 60.579) (width 0.35) (layer F.Cu) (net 6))
 (segment (start 86.106 59.578) (end 89.589 59.578) (width 0.35) (layer F.Cu) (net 6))
 (segment (start 86.106 59.578) (end 86.106 59.804) (width 0.35) (layer F.Cu) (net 6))
 (segment (start 86.868 60.579) (end 90.577 60.579) (width 0.35) (layer F.Cu) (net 6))
 (segment (start 86.106 59.804) (end 86.881 60.579) (width 0.35) (layer F.Cu) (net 6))
 (segment (start 86.106 58.039) (end 86.881 57.264) (width 0.35) (layer F.Cu) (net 7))
 (segment (start 86.106 58.054) (end 86.106 58.28) (width 0.35) (layer F.Cu) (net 7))
 (segment (start 89.576 58.278) (end 90.577 57.277) (width 0.35) (layer F.Cu) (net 7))
 (segment (start 86.106 58.278) (end 89.589 58.278) (width 0.35) (layer F.Cu) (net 7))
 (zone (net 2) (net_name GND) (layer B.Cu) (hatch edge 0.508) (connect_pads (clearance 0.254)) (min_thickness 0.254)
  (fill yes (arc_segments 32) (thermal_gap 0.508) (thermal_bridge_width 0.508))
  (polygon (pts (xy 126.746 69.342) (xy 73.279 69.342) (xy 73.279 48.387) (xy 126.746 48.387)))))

